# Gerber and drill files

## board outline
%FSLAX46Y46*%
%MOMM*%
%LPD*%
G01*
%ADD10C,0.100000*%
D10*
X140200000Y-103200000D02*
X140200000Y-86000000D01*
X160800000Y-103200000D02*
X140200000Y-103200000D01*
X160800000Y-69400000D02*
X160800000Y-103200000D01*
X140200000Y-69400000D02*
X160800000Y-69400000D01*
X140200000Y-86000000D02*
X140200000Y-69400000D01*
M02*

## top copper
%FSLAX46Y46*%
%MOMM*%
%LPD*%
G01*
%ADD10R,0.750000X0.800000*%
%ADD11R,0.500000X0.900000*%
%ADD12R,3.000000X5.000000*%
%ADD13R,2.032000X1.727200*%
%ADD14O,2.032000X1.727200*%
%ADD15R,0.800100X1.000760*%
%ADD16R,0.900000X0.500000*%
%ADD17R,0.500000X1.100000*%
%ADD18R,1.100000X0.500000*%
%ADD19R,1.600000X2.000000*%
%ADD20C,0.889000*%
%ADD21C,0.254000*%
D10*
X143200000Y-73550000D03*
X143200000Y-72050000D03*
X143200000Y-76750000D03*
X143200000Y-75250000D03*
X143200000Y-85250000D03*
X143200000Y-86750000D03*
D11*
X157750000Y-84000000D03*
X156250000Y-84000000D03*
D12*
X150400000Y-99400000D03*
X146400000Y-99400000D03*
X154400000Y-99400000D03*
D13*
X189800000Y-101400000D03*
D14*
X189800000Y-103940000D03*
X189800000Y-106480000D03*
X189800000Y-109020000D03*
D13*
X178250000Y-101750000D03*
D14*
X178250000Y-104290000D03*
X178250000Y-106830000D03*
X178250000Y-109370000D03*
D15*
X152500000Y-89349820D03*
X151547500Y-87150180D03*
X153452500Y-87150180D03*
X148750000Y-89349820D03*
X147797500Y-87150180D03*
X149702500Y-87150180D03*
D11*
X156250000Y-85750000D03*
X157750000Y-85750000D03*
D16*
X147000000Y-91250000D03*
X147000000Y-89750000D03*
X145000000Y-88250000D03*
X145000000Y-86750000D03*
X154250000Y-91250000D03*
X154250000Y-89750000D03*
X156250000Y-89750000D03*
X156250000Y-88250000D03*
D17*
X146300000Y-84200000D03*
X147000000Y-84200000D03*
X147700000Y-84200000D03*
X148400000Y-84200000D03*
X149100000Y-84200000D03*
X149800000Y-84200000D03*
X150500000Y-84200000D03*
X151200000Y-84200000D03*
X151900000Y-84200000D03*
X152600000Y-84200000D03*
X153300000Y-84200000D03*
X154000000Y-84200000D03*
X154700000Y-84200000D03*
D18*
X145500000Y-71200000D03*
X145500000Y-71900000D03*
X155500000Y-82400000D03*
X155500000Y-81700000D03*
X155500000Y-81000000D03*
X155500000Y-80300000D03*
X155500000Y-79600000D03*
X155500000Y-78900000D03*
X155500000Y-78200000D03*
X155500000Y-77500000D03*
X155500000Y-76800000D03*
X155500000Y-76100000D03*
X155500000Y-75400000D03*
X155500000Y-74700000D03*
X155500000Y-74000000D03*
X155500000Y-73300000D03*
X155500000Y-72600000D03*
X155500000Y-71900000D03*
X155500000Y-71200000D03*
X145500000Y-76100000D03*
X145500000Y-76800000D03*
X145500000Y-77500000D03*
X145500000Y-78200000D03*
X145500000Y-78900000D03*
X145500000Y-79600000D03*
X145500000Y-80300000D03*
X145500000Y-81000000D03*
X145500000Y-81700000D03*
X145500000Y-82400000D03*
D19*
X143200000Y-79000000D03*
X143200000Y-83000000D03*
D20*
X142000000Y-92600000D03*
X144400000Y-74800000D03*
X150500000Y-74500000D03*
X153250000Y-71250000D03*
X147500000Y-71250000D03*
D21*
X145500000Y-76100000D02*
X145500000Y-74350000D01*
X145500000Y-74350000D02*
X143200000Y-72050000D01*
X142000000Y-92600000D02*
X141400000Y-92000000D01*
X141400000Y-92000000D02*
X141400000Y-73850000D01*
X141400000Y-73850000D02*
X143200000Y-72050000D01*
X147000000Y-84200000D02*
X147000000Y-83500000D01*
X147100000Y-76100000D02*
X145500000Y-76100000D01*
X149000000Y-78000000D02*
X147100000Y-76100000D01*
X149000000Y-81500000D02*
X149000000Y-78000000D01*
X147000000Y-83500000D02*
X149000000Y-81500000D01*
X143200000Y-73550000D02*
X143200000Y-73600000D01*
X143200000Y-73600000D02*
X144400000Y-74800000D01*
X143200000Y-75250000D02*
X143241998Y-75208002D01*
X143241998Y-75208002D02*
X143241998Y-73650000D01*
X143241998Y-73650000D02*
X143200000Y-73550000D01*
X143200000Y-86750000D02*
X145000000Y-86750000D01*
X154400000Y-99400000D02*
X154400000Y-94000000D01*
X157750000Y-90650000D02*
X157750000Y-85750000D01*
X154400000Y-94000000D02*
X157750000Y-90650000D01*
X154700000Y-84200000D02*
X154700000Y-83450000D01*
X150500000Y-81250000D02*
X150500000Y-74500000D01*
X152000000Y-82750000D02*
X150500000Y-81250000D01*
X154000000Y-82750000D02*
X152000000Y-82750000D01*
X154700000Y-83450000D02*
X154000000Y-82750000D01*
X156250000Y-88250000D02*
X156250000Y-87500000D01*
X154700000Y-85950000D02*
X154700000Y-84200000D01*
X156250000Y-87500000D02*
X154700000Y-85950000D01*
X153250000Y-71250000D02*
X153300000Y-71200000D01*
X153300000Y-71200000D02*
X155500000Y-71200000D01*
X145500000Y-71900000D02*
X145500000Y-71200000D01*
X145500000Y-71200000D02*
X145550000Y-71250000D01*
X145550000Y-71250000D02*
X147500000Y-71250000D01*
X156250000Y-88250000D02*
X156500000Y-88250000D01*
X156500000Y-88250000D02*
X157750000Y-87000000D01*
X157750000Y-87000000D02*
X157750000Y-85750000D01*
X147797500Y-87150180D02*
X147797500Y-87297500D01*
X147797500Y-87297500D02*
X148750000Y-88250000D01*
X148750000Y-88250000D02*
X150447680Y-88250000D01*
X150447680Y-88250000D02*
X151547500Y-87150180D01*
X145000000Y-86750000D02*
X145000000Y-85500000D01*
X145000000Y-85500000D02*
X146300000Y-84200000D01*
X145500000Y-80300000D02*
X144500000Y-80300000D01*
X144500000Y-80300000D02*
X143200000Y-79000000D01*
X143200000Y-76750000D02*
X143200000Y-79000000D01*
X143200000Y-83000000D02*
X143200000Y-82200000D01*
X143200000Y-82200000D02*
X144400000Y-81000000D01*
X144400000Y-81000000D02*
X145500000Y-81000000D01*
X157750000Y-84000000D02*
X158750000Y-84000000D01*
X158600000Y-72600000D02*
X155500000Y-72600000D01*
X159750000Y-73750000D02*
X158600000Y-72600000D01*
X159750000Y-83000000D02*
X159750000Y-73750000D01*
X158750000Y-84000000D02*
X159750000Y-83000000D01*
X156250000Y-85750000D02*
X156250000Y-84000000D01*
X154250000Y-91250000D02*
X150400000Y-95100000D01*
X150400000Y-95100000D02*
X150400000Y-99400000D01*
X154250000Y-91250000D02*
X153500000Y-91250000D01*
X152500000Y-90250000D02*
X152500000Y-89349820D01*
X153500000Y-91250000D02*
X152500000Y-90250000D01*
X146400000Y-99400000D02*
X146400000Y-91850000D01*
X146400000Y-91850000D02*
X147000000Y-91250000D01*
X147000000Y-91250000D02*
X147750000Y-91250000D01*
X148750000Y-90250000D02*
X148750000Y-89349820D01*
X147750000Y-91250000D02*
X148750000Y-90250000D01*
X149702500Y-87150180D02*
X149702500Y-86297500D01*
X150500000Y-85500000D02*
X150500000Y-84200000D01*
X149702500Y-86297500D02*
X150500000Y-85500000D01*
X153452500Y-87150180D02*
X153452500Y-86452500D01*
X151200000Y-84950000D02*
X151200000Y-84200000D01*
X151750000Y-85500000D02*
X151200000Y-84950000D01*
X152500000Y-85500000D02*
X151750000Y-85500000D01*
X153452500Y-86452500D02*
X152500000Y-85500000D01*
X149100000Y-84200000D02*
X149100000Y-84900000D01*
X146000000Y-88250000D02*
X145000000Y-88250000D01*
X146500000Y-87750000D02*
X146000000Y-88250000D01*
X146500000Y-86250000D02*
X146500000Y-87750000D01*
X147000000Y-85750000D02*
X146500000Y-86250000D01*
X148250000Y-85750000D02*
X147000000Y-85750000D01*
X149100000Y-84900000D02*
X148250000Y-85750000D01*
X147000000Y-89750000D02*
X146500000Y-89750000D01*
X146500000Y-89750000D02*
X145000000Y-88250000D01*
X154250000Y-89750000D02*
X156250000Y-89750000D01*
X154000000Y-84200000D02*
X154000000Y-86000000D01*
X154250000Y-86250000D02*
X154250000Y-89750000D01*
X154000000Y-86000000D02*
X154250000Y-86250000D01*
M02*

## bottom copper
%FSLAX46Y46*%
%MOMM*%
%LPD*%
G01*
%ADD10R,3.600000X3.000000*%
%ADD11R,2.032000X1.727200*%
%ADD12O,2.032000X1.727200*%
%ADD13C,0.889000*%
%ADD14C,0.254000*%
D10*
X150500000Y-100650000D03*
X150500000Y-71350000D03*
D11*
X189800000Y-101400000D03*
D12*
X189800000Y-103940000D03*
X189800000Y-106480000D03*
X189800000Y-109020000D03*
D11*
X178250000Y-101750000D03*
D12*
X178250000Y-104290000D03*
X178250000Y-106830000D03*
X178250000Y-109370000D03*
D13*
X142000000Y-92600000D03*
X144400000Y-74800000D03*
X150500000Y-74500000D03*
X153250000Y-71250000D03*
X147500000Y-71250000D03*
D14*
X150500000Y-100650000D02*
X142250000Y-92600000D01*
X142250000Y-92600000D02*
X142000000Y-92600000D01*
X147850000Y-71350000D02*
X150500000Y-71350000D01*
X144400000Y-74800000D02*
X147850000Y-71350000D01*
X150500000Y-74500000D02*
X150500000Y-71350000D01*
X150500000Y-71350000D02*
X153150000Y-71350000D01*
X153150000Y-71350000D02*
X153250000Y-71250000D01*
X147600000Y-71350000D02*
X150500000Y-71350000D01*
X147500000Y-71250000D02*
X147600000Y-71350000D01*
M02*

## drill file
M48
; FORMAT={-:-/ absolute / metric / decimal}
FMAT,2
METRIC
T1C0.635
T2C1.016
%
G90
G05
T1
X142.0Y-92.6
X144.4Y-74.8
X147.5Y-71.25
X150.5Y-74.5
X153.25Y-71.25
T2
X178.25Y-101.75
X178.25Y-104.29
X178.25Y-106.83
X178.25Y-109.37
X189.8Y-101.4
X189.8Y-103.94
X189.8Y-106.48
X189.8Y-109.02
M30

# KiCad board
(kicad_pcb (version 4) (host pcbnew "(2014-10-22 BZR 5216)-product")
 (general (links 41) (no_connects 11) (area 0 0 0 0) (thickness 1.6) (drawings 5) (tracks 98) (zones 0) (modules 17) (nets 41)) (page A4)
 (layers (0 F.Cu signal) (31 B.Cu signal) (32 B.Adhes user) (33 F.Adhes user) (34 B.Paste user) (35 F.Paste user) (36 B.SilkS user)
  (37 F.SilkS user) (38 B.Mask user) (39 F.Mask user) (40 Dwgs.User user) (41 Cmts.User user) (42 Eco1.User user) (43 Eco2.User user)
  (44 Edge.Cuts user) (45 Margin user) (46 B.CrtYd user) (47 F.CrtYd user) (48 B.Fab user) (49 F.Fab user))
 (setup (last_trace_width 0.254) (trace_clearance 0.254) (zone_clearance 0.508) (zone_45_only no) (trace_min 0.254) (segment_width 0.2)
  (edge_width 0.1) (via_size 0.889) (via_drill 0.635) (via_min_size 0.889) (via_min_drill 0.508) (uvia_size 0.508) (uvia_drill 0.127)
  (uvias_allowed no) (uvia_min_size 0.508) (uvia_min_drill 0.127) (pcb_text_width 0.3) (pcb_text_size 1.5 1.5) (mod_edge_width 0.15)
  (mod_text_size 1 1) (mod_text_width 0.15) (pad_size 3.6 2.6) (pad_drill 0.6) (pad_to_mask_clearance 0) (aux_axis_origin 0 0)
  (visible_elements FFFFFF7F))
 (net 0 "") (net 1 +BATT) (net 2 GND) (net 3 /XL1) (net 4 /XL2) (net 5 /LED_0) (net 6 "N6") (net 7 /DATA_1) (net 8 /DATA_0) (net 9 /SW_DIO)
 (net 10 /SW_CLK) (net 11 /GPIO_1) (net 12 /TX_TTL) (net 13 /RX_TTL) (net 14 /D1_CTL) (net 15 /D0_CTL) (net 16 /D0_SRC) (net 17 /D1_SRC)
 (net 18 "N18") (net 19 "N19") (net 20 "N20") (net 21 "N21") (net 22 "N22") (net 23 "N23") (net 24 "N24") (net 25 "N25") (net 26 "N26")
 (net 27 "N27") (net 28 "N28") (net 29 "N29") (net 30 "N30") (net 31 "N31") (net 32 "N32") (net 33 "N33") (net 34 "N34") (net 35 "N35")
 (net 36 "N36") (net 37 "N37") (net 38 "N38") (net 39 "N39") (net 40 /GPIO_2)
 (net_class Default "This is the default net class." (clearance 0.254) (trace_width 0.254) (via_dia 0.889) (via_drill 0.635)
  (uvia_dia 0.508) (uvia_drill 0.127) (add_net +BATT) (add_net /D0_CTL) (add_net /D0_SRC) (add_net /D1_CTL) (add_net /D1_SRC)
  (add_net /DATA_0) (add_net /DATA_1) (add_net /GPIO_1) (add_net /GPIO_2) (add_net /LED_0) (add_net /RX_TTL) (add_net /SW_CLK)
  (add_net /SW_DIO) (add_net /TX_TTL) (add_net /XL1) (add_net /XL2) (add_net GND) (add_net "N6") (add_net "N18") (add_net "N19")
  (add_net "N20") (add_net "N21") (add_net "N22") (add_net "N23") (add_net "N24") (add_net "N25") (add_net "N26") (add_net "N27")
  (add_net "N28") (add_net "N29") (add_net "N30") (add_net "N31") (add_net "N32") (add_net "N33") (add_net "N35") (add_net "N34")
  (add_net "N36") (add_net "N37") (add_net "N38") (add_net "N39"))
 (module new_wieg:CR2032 (layer B.Cu) (at 150.5 86)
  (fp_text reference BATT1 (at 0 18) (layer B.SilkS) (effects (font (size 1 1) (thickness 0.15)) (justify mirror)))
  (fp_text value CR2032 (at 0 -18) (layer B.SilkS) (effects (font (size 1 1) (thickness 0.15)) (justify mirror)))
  (pad 1 smd rect (at 0 14.65) (size 3.6 3) (layers B.Cu B.Paste B.Mask) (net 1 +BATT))
  (pad 2 smd rect (at 0 -14.65) (size 3.6 3) (layers B.Cu B.Paste B.Mask) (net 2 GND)))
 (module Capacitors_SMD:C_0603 (layer F.Cu) (at 143.2 72.8 90)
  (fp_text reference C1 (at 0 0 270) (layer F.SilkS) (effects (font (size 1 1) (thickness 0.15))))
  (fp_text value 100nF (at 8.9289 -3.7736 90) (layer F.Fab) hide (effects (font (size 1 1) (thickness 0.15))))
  (pad 1 smd rect (at -0.75 0 90) (size 0.8 0.75) (layers F.Cu F.Paste F.Mask) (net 2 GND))
  (pad 2 smd rect (at 0.75 0 90) (size 0.8 0.75) (layers F.Cu F.Paste F.Mask) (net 1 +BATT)))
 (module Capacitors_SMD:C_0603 (layer F.Cu) (at 143.2 76 90)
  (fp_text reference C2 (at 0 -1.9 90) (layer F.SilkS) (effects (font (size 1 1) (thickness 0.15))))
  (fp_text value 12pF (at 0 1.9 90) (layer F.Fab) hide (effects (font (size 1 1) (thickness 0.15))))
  (pad 1 smd rect (at -0.75 0 90) (size 0.8 0.75) (layers F.Cu F.Paste F.Mask) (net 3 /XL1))
  (pad 2 smd rect (at 0.75 0 90) (size 0.8 0.75) (layers F.Cu F.Paste F.Mask) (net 2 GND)))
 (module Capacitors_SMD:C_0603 (layer F.Cu) (at 143.2 86 270)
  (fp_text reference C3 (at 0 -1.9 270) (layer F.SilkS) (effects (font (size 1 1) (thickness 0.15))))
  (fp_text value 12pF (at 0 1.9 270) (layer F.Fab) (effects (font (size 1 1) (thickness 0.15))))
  (pad 1 smd rect (at -0.75 0 270) (size 0.8 0.75) (layers F.Cu F.Paste F.Mask) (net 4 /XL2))
  (pad 2 smd rect (at 0.75 0 270) (size 0.8 0.75) (layers F.Cu F.Paste F.Mask) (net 2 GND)))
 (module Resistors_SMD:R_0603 (layer F.Cu) (at 157 84 180)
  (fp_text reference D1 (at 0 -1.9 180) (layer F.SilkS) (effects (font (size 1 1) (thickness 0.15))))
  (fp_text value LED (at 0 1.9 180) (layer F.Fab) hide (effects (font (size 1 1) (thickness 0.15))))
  (pad 1 smd rect (at -0.75 0 180) (size 0.5 0.9) (layers F.Cu F.Paste F.Mask) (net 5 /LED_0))
  (pad 2 smd rect (at 0.75 0 180) (size 0.5 0.9) (layers F.Cu F.Paste F.Mask) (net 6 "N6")))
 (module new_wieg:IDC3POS (layer F.Cu) (at 150.4 99.4)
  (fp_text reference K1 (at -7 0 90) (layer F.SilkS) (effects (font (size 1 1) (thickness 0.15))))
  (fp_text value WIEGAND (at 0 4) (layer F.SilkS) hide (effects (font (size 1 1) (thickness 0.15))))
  (pad 2 smd rect (at 0 0) (size 3 5) (layers F.Cu F.Paste F.Mask) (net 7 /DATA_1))
  (pad 1 smd rect (at -4 0) (size 3 5) (layers F.Cu F.Paste F.Mask) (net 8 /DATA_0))
  (pad 3 smd rect (at 4 0) (size 3 5) (layers F.Cu F.Paste F.Mask) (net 2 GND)))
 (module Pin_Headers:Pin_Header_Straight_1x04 (layer F.Cu) (at 189.8 101.4)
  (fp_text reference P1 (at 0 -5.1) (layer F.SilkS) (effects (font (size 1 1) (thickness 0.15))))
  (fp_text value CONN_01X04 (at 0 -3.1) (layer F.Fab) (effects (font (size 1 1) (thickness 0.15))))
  (pad 1 thru_hole rect (at 0 0) (size 2.032 1.7272) (drill 1.016) (layers *.Cu *.Mask F.SilkS) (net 1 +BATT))
  (pad 2 thru_hole oval (at 0 2.54) (size 2.032 1.7272) (drill 1.016) (layers *.Cu *.Mask F.SilkS) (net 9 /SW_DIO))
  (pad 3 thru_hole oval (at 0 5.08) (size 2.032 1.7272) (drill 1.016) (layers *.Cu *.Mask F.SilkS) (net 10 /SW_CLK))
  (pad 4 thru_hole oval (at 0 7.62) (size 2.032 1.7272) (drill 1.016) (layers *.Cu *.Mask F.SilkS) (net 2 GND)))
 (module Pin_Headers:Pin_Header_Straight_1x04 (layer F.Cu) (at 178.25 101.75)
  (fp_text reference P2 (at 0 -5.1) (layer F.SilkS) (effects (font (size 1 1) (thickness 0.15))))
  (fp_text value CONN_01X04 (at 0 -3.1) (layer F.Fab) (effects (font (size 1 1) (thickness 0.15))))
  (pad 1 thru_hole rect (at 0 0) (size 2.032 1.7272) (drill 1.016) (layers *.Cu *.Mask F.SilkS) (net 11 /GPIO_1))
  (pad 2 thru_hole oval (at 0 2.54) (size 2.032 1.7272) (drill 1.016) (layers *.Cu *.Mask F.SilkS) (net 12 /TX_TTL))
  (pad 3 thru_hole oval (at 0 5.08) (size 2.032 1.7272) (drill 1.016) (layers *.Cu *.Mask F.SilkS) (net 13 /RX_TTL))
  (pad 4 thru_hole oval (at 0 7.62) (size 2.032 1.7272) (drill 1.016) (layers *.Cu *.Mask F.SilkS) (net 2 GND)))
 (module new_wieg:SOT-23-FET (layer F.Cu) (at 152.5 88.25 180)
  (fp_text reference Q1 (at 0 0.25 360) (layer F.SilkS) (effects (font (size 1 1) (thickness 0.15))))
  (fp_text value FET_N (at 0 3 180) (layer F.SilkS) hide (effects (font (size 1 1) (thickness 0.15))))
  (pad D smd rect (at 0 -1.09982 180) (size 0.8001 1.00076) (layers F.Cu F.Paste F.Mask) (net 7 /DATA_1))
  (pad S smd rect (at 0.9525 1.09982 180) (size 0.8001 1.00076) (layers F.Cu F.Paste F.Mask) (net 2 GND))
  (pad G smd rect (at -0.9525 1.09982 180) (size 0.8001 1.00076) (layers F.Cu F.Paste F.Mask) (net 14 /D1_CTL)))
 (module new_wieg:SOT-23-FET (layer F.Cu) (at 148.75 88.25 180)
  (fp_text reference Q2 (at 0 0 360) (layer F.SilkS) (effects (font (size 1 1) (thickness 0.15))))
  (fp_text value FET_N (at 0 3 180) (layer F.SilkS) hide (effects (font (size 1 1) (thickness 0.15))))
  (pad D smd rect (at 0 -1.09982 180) (size 0.8001 1.00076) (layers F.Cu F.Paste F.Mask) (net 8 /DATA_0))
  (pad S smd rect (at 0.9525 1.09982 180) (size 0.8001 1.00076) (layers F.Cu F.Paste F.Mask) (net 2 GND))
  (pad G smd rect (at -0.9525 1.09982 180) (size 0.8001 1.00076) (layers F.Cu F.Paste F.Mask) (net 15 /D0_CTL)))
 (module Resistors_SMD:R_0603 (layer F.Cu) (at 157 85.75)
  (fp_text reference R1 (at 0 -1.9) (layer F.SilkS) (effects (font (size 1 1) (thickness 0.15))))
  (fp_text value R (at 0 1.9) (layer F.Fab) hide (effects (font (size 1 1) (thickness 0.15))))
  (pad 1 smd rect (at -0.75 0) (size 0.5 0.9) (layers F.Cu F.Paste F.Mask) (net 6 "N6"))
  (pad 2 smd rect (at 0.75 0) (size 0.5 0.9) (layers F.Cu F.Paste F.Mask) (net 2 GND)))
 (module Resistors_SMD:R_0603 (layer F.Cu) (at 147 90.5 90)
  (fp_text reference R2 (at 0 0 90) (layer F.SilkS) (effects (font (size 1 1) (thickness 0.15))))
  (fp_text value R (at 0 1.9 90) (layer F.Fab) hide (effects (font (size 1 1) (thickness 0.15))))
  (pad 1 smd rect (at -0.75 0 90) (size 0.5 0.9) (layers F.Cu F.Paste F.Mask) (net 8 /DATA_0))
  (pad 2 smd rect (at 0.75 0 90) (size 0.5 0.9) (layers F.Cu F.Paste F.Mask) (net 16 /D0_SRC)))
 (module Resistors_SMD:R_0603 (layer F.Cu) (at 145 87.5 90)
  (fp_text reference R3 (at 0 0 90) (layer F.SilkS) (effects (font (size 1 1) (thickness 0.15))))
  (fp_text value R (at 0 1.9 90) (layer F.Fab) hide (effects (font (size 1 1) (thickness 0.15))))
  (pad 1 smd rect (at -0.75 0 90) (size 0.5 0.9) (layers F.Cu F.Paste F.Mask) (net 16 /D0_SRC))
  (pad 2 smd rect (at 0.75 0 90) (size 0.5 0.9) (layers F.Cu F.Paste F.Mask) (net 2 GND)))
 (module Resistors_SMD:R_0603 (layer F.Cu) (at 154.25 90.5 90)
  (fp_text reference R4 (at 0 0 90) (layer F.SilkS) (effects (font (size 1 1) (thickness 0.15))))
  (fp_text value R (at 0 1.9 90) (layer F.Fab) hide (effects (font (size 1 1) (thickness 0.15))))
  (pad 1 smd rect (at -0.75 0 90) (size 0.5 0.9) (layers F.Cu F.Paste F.Mask) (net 7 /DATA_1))
  (pad 2 smd rect (at 0.75 0 90) (size 0.5 0.9) (layers F.Cu F.Paste F.Mask) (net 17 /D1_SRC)))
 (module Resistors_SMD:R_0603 (layer F.Cu) (at 156.25 89 90)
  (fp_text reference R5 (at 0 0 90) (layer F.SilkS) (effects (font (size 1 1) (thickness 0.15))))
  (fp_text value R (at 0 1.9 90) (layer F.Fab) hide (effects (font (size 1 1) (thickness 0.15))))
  (pad 1 smd rect (at -0.75 0 90) (size 0.5 0.9) (layers F.Cu F.Paste F.Mask) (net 17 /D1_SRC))
  (pad 2 smd rect (at 0.75 0 90) (size 0.5 0.9) (layers F.Cu F.Paste F.Mask) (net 2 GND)))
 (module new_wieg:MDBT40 (layer F.Cu) (at 150.5 84.2)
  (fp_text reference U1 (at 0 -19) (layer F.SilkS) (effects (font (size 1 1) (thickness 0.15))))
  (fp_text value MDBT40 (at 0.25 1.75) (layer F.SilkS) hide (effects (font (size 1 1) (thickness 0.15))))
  (pad 13 smd rect (at -4.2 0) (size 0.5 1.1) (layers F.Cu F.Paste F.Mask) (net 2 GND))
  (pad 14 smd rect (at -3.5 0) (size 0.5 1.1) (layers F.Cu F.Paste F.Mask) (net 1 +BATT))
  (pad 15 smd rect (at -2.8 0) (size 0.5 1.1) (layers F.Cu F.Paste F.Mask) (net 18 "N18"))
  (pad 16 smd rect (at -2.1 0) (size 0.5 1.1) (layers F.Cu F.Paste F.Mask) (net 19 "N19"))
  (pad 17 smd rect (at -1.4 0) (size 0.5 1.1) (layers F.Cu F.Paste F.Mask) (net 16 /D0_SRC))
  (pad 18 smd rect (at -0.7 0) (size 0.5 1.1) (layers F.Cu F.Paste F.Mask) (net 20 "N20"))
  (pad 19 smd rect (at 0 0) (size 0.5 1.1) (layers F.Cu F.Paste F.Mask) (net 15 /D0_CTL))
  (pad 20 smd rect (at 0.7 0) (size 0.5 1.1) (layers F.Cu F.Paste F.Mask) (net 14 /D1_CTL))
  (pad 21 smd rect (at 1.4 0) (size 0.5 1.1) (layers F.Cu F.Paste F.Mask) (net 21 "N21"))
  (pad 22 smd rect (at 2.1 0) (size 0.5 1.1) (layers F.Cu F.Paste F.Mask) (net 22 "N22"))
  (pad 23 smd rect (at 2.8 0) (size 0.5 1.1) (layers F.Cu F.Paste F.Mask) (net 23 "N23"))
  (pad 24 smd rect (at 3.5 0) (size 0.5 1.1) (layers F.Cu F.Paste F.Mask) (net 17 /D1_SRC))
  (pad 25 smd rect (at 4.2 0) (size 0.5 1.1) (layers F.Cu F.Paste F.Mask) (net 2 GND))
  (pad 1 smd rect (at -5 -13) (size 1.1 0.5) (layers F.Cu F.Paste F.Mask) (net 2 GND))
  (pad 2 smd rect (at -5 -12.3) (size 1.1 0.5) (layers F.Cu F.Paste F.Mask) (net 2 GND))
  (pad 26 smd rect (at 5 -1.8) (size 1.1 0.5) (layers F.Cu F.Paste F.Mask) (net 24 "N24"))
  (pad 27 smd rect (at 5 -2.5) (size 1.1 0.5) (layers F.Cu F.Paste F.Mask) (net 12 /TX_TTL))
  (pad 28 smd rect (at 5 -3.2) (size 1.1 0.5) (layers F.Cu F.Paste F.Mask) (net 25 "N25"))
  (pad 29 smd rect (at 5 -3.9) (size 1.1 0.5) (layers F.Cu F.Paste F.Mask) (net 13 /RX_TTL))
  (pad 30 smd rect (at 5 -4.6) (size 1.1 0.5) (layers F.Cu F.Paste F.Mask) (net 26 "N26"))
  (pad 31 smd rect (at 5 -5.3) (size 1.1 0.5) (layers F.Cu F.Paste F.Mask) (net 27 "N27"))
  (pad 32 smd rect (at 5 -6) (size 1.1 0.5) (layers F.Cu F.Paste F.Mask) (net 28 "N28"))
  (pad 33 smd rect (at 5 -6.7) (size 1.1 0.5) (layers F.Cu F.Paste F.Mask) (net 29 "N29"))
  (pad 34 smd rect (at 5 -7.4) (size 1.1 0.5) (layers F.Cu F.Paste F.Mask) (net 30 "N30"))
  (pad 35 smd rect (at 5 -8.1) (size 1.1 0.5) (layers F.Cu F.Paste F.Mask) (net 9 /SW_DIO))
  (pad 36 smd rect (at 5 -8.8) (size 1.1 0.5) (layers F.Cu F.Paste F.Mask) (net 10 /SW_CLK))
  (pad 37 smd rect (at 5 -9.5) (size 1.1 0.5) (layers F.Cu F.Paste F.Mask) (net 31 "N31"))
  (pad 38 smd rect (at 5 -10.2) (size 1.1 0.5) (layers F.Cu F.Paste F.Mask) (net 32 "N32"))
  (pad 39 smd rect (at 5 -10.9) (size 1.1 0.5) (layers F.Cu F.Paste F.Mask) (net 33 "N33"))
  (pad 40 smd rect (at 5 -11.6) (size 1.1 0.5) (layers F.Cu F.Paste F.Mask) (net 5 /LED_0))
  (pad 41 smd rect (at 5 -12.3) (size 1.1 0.5) (layers F.Cu F.Paste F.Mask) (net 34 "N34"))
  (pad 42 smd rect (at 5 -13) (size 1.1 0.5) (layers F.Cu F.Paste F.Mask) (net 2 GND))
  (pad 3 smd rect (at -5 -8.1) (size 1.1 0.5) (layers F.Cu F.Paste F.Mask) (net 1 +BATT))
  (pad 4 smd rect (at -5 -7.4) (size 1.1 0.5) (layers F.Cu F.Paste F.Mask) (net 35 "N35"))
  (pad 5 smd rect (at -5 -6.7) (size 1.1 0.5) (layers F.Cu F.Paste F.Mask) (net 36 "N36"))
  (pad 6 smd rect (at -5 -6) (size 1.1 0.5) (layers F.Cu F.Paste F.Mask) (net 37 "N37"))
  (pad 7 smd rect (at -5 -5.3) (size 1.1 0.5) (layers F.Cu F.Paste F.Mask) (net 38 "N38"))
  (pad 8 smd rect (at -5 -4.6) (size 1.1 0.5) (layers F.Cu F.Paste F.Mask) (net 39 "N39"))
  (pad 9 smd rect (at -5 -3.9) (size 1.1 0.5) (layers F.Cu F.Paste F.Mask) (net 3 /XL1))
  (pad 10 smd rect (at -5 -3.2) (size 1.1 0.5) (layers F.Cu F.Paste F.Mask) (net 4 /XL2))
  (pad 11 smd rect (at -5 -2.5) (size 1.1 0.5) (layers F.Cu F.Paste F.Mask) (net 11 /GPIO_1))
  (pad 12 smd rect (at -5 -1.8) (size 1.1 0.5) (layers F.Cu F.Paste F.Mask) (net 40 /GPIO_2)))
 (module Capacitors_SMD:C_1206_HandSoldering (layer F.Cu) (at 143.2 81 270)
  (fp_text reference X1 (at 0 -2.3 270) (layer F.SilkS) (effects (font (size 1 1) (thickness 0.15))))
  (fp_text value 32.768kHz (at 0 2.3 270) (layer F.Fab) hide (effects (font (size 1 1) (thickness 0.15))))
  (pad 1 smd rect (at -2 0 270) (size 2 1.6) (layers F.Cu F.Paste F.Mask) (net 3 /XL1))
  (pad 2 smd rect (at 2 0 270) (size 2 1.6) (layers F.Cu F.Paste F.Mask) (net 4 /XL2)))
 (gr_line (start 140.2 103.2) (end 140.2 86) (angle 90) (layer Edge.Cuts) (width 0.1))
 (gr_line (start 160.8 103.2) (end 140.2 103.2) (angle 90) (layer Edge.Cuts) (width 0.1))
 (gr_line (start 160.8 69.4) (end 160.8 103.2) (angle 90) (layer Edge.Cuts) (width 0.1))
 (gr_line (start 140.2 69.4) (end 160.8 69.4) (angle 90) (layer Edge.Cuts) (width 0.1))
 (gr_line (start 140.2 86) (end 140.2 69.4) (angle 90) (layer Edge.Cuts) (width 0.1))
 (segment (start 145.5 76.1) (end 145.5 74.35) (width 0.254) (layer F.Cu) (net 1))
 (segment (start 145.5 74.35) (end 143.2 72.05) (width 0.254) (layer F.Cu) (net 1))
 (segment (start 142 92.6) (end 141.4 92) (width 0.254) (layer F.Cu) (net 1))
 (segment (start 141.4 92) (end 141.4 73.85) (width 0.254) (layer F.Cu) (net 1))
 (segment (start 141.4 73.85) (end 143.2 72.05) (width 0.254) (layer F.Cu) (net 1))
 (segment (start 150.5 100.65) (end 142.25 92.6) (width 0.254) (layer B.Cu) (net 1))
 (segment (start 142.25 92.6) (end 142 92.6) (width 0.254) (layer B.Cu) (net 1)) (via (at 142 92.6) (size 0.889) (layers F.Cu B.Cu) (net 1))
 (segment (start 147 84.2) (end 147 83.5) (width 0.254) (layer F.Cu) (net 1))
 (segment (start 147.1 76.1) (end 145.5 76.1) (width 0.254) (layer F.Cu) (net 1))
 (segment (start 149 78) (end 147.1 76.1) (width 0.254) (layer F.Cu) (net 1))
 (segment (start 149 81.5) (end 149 78) (width 0.254) (layer F.Cu) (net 1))
 (segment (start 147 83.5) (end 149 81.5) (width 0.254) (layer F.Cu) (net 1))
 (segment (start 143.2 73.55) (end 143.2 73.6) (width 0.254) (layer F.Cu) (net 2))
 (segment (start 143.2 73.6) (end 144.4 74.8) (width 0.254) (layer F.Cu) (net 2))
 (segment (start 147.85 71.35) (end 150.5 71.35) (width 0.254) (layer B.Cu) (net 2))
 (segment (start 144.4 74.8) (end 147.85 71.35) (width 0.254) (layer B.Cu) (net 2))
 (via (at 144.4 74.8) (size 0.889) (layers F.Cu B.Cu) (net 2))
 (segment (start 143.2 75.25) (end 143.241998 75.208002) (width 0.254) (layer F.Cu) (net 2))
 (segment (start 143.241998 75.208002) (end 143.241998 73.65) (width 0.254) (layer F.Cu) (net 2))
 (segment (start 143.241998 73.65) (end 143.2 73.55) (width 0.254) (layer F.Cu) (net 2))
 (segment (start 143.2 86.75) (end 145 86.75) (width 0.254) (layer F.Cu) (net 2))
 (segment (start 154.4 99.4) (end 154.4 94) (width 0.254) (layer F.Cu) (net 2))
 (segment (start 157.75 90.65) (end 157.75 85.75) (width 0.254) (layer F.Cu) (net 2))
 (segment (start 154.4 94) (end 157.75 90.65) (width 0.254) (layer F.Cu) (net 2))
 (segment (start 154.7 84.2) (end 154.7 83.45) (width 0.254) (layer F.Cu) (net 2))
 (segment (start 150.5 74.5) (end 150.5 71.35) (width 0.254) (layer B.Cu) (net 2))
 (via (at 150.5 74.5) (size 0.889) (layers F.Cu B.Cu) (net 2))
 (segment (start 150.5 81.25) (end 150.5 74.5) (width 0.254) (layer F.Cu) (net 2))
 (segment (start 152 82.75) (end 150.5 81.25) (width 0.254) (layer F.Cu) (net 2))
 (segment (start 154 82.75) (end 152 82.75) (width 0.254) (layer F.Cu) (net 2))
 (segment (start 154.7 83.45) (end 154 82.75) (width 0.254) (layer F.Cu) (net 2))
 (segment (start 156.25 88.25) (end 156.25 87.5) (width 0.254) (layer F.Cu) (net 2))
 (segment (start 154.7 85.95) (end 154.7 84.2) (width 0.254) (layer F.Cu) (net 2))
 (segment (start 156.25 87.5) (end 154.7 85.95) (width 0.254) (layer F.Cu) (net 2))
 (segment (start 150.5 71.35) (end 153.15 71.35) (width 0.254) (layer B.Cu) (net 2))
 (segment (start 153.15 71.35) (end 153.25 71.25) (width 0.254) (layer B.Cu) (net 2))
 (via (at 153.25 71.25) (size 0.889) (layers F.Cu B.Cu) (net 2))
 (segment (start 153.25 71.25) (end 153.3 71.2) (width 0.254) (layer F.Cu) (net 2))
 (segment (start 153.3 71.2) (end 155.5 71.2) (width 0.254) (layer F.Cu) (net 2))
 (segment (start 145.5 71.9) (end 145.5 71.2) (width 0.254) (layer F.Cu) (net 2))
 (segment (start 145.5 71.2) (end 145.55 71.25) (width 0.254) (layer F.Cu) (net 2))
 (segment (start 145.55 71.25) (end 147.5 71.25) (width 0.254) (layer F.Cu) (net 2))
 (segment (start 147.6 71.35) (end 150.5 71.35) (width 0.254) (layer B.Cu) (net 2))
 (segment (start 147.5 71.25) (end 147.6 71.35) (width 0.254) (layer B.Cu) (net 2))
 (via (at 147.5 71.25) (size 0.889) (layers F.Cu B.Cu) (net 2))
 (segment (start 156.25 88.25) (end 156.5 88.25) (width 0.254) (layer F.Cu) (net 2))
 (segment (start 156.5 88.25) (end 157.75 87) (width 0.254) (layer F.Cu) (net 2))
 (segment (start 157.75 87) (end 157.75 85.75) (width 0.254) (layer F.Cu) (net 2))
 (segment (start 147.7975 87.15018) (end 147.7975 87.2975) (width 0.254) (layer F.Cu) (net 2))
 (segment (start 147.7975 87.2975) (end 148.75 88.25) (width 0.254) (layer F.Cu) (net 2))
 (segment (start 148.75 88.25) (end 150.44768 88.25) (width 0.254) (layer F.Cu) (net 2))
 (segment (start 150.44768 88.25) (end 151.5475 87.15018) (width 0.254) (layer F.Cu) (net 2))
 (segment (start 145 86.75) (end 145 85.5) (width 0.254) (layer F.Cu) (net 2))
 (segment (start 145 85.5) (end 146.3 84.2) (width 0.254) (layer F.Cu) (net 2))
 (segment (start 145.5 80.3) (end 144.5 80.3) (width 0.254) (layer F.Cu) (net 3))
 (segment (start 144.5 80.3) (end 143.2 79) (width 0.254) (layer F.Cu) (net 3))
 (segment (start 143.2 76.75) (end 143.2 79) (width 0.254) (layer F.Cu) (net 3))
 (segment (start 143.2 83) (end 143.2 82.2) (width 0.254) (layer F.Cu) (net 4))
 (segment (start 143.2 82.2) (end 144.4 81) (width 0.254) (layer F.Cu) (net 4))
 (segment (start 144.4 81) (end 145.5 81) (width 0.254) (layer F.Cu) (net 4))
 (segment (start 157.75 84) (end 158.75 84) (width 0.254) (layer F.Cu) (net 5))
 (segment (start 158.6 72.6) (end 155.5 72.6) (width 0.254) (layer F.Cu) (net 5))
 (segment (start 159.75 73.75) (end 158.6 72.6) (width 0.254) (layer F.Cu) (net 5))
 (segment (start 159.75 83) (end 159.75 73.75) (width 0.254) (layer F.Cu) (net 5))
 (segment (start 158.75 84) (end 159.75 83) (width 0.254) (layer F.Cu) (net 5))
 (segment (start 156.25 85.75) (end 156.25 84) (width 0.254) (layer F.Cu) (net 6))
 (segment (start 154.25 91.25) (end 150.4 95.1) (width 0.254) (layer F.Cu) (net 7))
 (segment (start 150.4 95.1) (end 150.4 99.4) (width 0.254) (layer F.Cu) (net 7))
 (segment (start 154.25 91.25) (end 153.5 91.25) (width 0.254) (layer F.Cu) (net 7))
 (segment (start 152.5 90.25) (end 152.5 89.34982) (width 0.254) (layer F.Cu) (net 7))
 (segment (start 153.5 91.25) (end 152.5 90.25) (width 0.254) (layer F.Cu) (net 7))
 (segment (start 146.4 99.4) (end 146.4 91.85) (width 0.254) (layer F.Cu) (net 8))
 (segment (start 146.4 91.85) (end 147 91.25) (width 0.254) (layer F.Cu) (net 8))
 (segment (start 147 91.25) (end 147.75 91.25) (width 0.254) (layer F.Cu) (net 8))
 (segment (start 148.75 90.25) (end 148.75 89.34982) (width 0.254) (layer F.Cu) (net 8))
 (segment (start 147.75 91.25) (end 148.75 90.25) (width 0.254) (layer F.Cu) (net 8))
 (segment (start 149.7025 87.15018) (end 149.7025 86.2975) (width 0.254) (layer F.Cu) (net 15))
 (segment (start 150.5 85.5) (end 150.5 84.2) (width 0.254) (layer F.Cu) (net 15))
 (segment (start 149.7025 86.2975) (end 150.5 85.5) (width 0.254) (layer F.Cu) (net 15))
 (segment (start 153.4525 87.15018) (end 153.4525 86.4525) (width 0.254) (layer F.Cu) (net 14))
 (segment (start 151.2 84.95) (end 151.2 84.2) (width 0.254) (layer F.Cu) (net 14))
 (segment (start 151.75 85.5) (end 151.2 84.95) (width 0.254) (layer F.Cu) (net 14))
 (segment (start 152.5 85.5) (end 151.75 85.5) (width 0.254) (layer F.Cu) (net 14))
 (segment (start 153.4525 86.4525) (end 152.5 85.5) (width 0.254) (layer F.Cu) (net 14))
 (segment (start 149.1 84.2) (end 149.1 84.9) (width 0.254) (layer F.Cu) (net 16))
 (segment (start 146 88.25) (end 145 88.25) (width 0.254) (layer F.Cu) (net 16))
 (segment (start 146.5 87.75) (end 146 88.25) (width 0.254) (layer F.Cu) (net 16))
 (segment (start 146.5 86.25) (end 146.5 87.75) (width 0.254) (layer F.Cu) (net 16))
 (segment (start 147 85.75) (end 146.5 86.25) (width 0.254) (layer F.Cu) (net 16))
 (segment (start 148.25 85.75) (end 147 85.75) (width 0.254) (layer F.Cu) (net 16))
 (segment (start 149.1 84.9) (end 148.25 85.75) (width 0.254) (layer F.Cu) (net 16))
 (segment (start 147 89.75) (end 146.5 89.75) (width 0.254) (layer F.Cu) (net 16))
 (segment (start 146.5 89.75) (end 145 88.25) (width 0.254) (layer F.Cu) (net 16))
 (segment (start 154.25 89.75) (end 156.25 89.75) (width 0.254) (layer F.Cu) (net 17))
 (segment (start 154 84.2) (end 154 86) (width 0.254) (layer F.Cu) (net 17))
 (segment (start 154.25 86.25) (end 154.25 89.75) (width 0.254) (layer F.Cu) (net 17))
 (segment (start 154 86) (end 154.25 86.25) (width 0.254) (layer F.Cu) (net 17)))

